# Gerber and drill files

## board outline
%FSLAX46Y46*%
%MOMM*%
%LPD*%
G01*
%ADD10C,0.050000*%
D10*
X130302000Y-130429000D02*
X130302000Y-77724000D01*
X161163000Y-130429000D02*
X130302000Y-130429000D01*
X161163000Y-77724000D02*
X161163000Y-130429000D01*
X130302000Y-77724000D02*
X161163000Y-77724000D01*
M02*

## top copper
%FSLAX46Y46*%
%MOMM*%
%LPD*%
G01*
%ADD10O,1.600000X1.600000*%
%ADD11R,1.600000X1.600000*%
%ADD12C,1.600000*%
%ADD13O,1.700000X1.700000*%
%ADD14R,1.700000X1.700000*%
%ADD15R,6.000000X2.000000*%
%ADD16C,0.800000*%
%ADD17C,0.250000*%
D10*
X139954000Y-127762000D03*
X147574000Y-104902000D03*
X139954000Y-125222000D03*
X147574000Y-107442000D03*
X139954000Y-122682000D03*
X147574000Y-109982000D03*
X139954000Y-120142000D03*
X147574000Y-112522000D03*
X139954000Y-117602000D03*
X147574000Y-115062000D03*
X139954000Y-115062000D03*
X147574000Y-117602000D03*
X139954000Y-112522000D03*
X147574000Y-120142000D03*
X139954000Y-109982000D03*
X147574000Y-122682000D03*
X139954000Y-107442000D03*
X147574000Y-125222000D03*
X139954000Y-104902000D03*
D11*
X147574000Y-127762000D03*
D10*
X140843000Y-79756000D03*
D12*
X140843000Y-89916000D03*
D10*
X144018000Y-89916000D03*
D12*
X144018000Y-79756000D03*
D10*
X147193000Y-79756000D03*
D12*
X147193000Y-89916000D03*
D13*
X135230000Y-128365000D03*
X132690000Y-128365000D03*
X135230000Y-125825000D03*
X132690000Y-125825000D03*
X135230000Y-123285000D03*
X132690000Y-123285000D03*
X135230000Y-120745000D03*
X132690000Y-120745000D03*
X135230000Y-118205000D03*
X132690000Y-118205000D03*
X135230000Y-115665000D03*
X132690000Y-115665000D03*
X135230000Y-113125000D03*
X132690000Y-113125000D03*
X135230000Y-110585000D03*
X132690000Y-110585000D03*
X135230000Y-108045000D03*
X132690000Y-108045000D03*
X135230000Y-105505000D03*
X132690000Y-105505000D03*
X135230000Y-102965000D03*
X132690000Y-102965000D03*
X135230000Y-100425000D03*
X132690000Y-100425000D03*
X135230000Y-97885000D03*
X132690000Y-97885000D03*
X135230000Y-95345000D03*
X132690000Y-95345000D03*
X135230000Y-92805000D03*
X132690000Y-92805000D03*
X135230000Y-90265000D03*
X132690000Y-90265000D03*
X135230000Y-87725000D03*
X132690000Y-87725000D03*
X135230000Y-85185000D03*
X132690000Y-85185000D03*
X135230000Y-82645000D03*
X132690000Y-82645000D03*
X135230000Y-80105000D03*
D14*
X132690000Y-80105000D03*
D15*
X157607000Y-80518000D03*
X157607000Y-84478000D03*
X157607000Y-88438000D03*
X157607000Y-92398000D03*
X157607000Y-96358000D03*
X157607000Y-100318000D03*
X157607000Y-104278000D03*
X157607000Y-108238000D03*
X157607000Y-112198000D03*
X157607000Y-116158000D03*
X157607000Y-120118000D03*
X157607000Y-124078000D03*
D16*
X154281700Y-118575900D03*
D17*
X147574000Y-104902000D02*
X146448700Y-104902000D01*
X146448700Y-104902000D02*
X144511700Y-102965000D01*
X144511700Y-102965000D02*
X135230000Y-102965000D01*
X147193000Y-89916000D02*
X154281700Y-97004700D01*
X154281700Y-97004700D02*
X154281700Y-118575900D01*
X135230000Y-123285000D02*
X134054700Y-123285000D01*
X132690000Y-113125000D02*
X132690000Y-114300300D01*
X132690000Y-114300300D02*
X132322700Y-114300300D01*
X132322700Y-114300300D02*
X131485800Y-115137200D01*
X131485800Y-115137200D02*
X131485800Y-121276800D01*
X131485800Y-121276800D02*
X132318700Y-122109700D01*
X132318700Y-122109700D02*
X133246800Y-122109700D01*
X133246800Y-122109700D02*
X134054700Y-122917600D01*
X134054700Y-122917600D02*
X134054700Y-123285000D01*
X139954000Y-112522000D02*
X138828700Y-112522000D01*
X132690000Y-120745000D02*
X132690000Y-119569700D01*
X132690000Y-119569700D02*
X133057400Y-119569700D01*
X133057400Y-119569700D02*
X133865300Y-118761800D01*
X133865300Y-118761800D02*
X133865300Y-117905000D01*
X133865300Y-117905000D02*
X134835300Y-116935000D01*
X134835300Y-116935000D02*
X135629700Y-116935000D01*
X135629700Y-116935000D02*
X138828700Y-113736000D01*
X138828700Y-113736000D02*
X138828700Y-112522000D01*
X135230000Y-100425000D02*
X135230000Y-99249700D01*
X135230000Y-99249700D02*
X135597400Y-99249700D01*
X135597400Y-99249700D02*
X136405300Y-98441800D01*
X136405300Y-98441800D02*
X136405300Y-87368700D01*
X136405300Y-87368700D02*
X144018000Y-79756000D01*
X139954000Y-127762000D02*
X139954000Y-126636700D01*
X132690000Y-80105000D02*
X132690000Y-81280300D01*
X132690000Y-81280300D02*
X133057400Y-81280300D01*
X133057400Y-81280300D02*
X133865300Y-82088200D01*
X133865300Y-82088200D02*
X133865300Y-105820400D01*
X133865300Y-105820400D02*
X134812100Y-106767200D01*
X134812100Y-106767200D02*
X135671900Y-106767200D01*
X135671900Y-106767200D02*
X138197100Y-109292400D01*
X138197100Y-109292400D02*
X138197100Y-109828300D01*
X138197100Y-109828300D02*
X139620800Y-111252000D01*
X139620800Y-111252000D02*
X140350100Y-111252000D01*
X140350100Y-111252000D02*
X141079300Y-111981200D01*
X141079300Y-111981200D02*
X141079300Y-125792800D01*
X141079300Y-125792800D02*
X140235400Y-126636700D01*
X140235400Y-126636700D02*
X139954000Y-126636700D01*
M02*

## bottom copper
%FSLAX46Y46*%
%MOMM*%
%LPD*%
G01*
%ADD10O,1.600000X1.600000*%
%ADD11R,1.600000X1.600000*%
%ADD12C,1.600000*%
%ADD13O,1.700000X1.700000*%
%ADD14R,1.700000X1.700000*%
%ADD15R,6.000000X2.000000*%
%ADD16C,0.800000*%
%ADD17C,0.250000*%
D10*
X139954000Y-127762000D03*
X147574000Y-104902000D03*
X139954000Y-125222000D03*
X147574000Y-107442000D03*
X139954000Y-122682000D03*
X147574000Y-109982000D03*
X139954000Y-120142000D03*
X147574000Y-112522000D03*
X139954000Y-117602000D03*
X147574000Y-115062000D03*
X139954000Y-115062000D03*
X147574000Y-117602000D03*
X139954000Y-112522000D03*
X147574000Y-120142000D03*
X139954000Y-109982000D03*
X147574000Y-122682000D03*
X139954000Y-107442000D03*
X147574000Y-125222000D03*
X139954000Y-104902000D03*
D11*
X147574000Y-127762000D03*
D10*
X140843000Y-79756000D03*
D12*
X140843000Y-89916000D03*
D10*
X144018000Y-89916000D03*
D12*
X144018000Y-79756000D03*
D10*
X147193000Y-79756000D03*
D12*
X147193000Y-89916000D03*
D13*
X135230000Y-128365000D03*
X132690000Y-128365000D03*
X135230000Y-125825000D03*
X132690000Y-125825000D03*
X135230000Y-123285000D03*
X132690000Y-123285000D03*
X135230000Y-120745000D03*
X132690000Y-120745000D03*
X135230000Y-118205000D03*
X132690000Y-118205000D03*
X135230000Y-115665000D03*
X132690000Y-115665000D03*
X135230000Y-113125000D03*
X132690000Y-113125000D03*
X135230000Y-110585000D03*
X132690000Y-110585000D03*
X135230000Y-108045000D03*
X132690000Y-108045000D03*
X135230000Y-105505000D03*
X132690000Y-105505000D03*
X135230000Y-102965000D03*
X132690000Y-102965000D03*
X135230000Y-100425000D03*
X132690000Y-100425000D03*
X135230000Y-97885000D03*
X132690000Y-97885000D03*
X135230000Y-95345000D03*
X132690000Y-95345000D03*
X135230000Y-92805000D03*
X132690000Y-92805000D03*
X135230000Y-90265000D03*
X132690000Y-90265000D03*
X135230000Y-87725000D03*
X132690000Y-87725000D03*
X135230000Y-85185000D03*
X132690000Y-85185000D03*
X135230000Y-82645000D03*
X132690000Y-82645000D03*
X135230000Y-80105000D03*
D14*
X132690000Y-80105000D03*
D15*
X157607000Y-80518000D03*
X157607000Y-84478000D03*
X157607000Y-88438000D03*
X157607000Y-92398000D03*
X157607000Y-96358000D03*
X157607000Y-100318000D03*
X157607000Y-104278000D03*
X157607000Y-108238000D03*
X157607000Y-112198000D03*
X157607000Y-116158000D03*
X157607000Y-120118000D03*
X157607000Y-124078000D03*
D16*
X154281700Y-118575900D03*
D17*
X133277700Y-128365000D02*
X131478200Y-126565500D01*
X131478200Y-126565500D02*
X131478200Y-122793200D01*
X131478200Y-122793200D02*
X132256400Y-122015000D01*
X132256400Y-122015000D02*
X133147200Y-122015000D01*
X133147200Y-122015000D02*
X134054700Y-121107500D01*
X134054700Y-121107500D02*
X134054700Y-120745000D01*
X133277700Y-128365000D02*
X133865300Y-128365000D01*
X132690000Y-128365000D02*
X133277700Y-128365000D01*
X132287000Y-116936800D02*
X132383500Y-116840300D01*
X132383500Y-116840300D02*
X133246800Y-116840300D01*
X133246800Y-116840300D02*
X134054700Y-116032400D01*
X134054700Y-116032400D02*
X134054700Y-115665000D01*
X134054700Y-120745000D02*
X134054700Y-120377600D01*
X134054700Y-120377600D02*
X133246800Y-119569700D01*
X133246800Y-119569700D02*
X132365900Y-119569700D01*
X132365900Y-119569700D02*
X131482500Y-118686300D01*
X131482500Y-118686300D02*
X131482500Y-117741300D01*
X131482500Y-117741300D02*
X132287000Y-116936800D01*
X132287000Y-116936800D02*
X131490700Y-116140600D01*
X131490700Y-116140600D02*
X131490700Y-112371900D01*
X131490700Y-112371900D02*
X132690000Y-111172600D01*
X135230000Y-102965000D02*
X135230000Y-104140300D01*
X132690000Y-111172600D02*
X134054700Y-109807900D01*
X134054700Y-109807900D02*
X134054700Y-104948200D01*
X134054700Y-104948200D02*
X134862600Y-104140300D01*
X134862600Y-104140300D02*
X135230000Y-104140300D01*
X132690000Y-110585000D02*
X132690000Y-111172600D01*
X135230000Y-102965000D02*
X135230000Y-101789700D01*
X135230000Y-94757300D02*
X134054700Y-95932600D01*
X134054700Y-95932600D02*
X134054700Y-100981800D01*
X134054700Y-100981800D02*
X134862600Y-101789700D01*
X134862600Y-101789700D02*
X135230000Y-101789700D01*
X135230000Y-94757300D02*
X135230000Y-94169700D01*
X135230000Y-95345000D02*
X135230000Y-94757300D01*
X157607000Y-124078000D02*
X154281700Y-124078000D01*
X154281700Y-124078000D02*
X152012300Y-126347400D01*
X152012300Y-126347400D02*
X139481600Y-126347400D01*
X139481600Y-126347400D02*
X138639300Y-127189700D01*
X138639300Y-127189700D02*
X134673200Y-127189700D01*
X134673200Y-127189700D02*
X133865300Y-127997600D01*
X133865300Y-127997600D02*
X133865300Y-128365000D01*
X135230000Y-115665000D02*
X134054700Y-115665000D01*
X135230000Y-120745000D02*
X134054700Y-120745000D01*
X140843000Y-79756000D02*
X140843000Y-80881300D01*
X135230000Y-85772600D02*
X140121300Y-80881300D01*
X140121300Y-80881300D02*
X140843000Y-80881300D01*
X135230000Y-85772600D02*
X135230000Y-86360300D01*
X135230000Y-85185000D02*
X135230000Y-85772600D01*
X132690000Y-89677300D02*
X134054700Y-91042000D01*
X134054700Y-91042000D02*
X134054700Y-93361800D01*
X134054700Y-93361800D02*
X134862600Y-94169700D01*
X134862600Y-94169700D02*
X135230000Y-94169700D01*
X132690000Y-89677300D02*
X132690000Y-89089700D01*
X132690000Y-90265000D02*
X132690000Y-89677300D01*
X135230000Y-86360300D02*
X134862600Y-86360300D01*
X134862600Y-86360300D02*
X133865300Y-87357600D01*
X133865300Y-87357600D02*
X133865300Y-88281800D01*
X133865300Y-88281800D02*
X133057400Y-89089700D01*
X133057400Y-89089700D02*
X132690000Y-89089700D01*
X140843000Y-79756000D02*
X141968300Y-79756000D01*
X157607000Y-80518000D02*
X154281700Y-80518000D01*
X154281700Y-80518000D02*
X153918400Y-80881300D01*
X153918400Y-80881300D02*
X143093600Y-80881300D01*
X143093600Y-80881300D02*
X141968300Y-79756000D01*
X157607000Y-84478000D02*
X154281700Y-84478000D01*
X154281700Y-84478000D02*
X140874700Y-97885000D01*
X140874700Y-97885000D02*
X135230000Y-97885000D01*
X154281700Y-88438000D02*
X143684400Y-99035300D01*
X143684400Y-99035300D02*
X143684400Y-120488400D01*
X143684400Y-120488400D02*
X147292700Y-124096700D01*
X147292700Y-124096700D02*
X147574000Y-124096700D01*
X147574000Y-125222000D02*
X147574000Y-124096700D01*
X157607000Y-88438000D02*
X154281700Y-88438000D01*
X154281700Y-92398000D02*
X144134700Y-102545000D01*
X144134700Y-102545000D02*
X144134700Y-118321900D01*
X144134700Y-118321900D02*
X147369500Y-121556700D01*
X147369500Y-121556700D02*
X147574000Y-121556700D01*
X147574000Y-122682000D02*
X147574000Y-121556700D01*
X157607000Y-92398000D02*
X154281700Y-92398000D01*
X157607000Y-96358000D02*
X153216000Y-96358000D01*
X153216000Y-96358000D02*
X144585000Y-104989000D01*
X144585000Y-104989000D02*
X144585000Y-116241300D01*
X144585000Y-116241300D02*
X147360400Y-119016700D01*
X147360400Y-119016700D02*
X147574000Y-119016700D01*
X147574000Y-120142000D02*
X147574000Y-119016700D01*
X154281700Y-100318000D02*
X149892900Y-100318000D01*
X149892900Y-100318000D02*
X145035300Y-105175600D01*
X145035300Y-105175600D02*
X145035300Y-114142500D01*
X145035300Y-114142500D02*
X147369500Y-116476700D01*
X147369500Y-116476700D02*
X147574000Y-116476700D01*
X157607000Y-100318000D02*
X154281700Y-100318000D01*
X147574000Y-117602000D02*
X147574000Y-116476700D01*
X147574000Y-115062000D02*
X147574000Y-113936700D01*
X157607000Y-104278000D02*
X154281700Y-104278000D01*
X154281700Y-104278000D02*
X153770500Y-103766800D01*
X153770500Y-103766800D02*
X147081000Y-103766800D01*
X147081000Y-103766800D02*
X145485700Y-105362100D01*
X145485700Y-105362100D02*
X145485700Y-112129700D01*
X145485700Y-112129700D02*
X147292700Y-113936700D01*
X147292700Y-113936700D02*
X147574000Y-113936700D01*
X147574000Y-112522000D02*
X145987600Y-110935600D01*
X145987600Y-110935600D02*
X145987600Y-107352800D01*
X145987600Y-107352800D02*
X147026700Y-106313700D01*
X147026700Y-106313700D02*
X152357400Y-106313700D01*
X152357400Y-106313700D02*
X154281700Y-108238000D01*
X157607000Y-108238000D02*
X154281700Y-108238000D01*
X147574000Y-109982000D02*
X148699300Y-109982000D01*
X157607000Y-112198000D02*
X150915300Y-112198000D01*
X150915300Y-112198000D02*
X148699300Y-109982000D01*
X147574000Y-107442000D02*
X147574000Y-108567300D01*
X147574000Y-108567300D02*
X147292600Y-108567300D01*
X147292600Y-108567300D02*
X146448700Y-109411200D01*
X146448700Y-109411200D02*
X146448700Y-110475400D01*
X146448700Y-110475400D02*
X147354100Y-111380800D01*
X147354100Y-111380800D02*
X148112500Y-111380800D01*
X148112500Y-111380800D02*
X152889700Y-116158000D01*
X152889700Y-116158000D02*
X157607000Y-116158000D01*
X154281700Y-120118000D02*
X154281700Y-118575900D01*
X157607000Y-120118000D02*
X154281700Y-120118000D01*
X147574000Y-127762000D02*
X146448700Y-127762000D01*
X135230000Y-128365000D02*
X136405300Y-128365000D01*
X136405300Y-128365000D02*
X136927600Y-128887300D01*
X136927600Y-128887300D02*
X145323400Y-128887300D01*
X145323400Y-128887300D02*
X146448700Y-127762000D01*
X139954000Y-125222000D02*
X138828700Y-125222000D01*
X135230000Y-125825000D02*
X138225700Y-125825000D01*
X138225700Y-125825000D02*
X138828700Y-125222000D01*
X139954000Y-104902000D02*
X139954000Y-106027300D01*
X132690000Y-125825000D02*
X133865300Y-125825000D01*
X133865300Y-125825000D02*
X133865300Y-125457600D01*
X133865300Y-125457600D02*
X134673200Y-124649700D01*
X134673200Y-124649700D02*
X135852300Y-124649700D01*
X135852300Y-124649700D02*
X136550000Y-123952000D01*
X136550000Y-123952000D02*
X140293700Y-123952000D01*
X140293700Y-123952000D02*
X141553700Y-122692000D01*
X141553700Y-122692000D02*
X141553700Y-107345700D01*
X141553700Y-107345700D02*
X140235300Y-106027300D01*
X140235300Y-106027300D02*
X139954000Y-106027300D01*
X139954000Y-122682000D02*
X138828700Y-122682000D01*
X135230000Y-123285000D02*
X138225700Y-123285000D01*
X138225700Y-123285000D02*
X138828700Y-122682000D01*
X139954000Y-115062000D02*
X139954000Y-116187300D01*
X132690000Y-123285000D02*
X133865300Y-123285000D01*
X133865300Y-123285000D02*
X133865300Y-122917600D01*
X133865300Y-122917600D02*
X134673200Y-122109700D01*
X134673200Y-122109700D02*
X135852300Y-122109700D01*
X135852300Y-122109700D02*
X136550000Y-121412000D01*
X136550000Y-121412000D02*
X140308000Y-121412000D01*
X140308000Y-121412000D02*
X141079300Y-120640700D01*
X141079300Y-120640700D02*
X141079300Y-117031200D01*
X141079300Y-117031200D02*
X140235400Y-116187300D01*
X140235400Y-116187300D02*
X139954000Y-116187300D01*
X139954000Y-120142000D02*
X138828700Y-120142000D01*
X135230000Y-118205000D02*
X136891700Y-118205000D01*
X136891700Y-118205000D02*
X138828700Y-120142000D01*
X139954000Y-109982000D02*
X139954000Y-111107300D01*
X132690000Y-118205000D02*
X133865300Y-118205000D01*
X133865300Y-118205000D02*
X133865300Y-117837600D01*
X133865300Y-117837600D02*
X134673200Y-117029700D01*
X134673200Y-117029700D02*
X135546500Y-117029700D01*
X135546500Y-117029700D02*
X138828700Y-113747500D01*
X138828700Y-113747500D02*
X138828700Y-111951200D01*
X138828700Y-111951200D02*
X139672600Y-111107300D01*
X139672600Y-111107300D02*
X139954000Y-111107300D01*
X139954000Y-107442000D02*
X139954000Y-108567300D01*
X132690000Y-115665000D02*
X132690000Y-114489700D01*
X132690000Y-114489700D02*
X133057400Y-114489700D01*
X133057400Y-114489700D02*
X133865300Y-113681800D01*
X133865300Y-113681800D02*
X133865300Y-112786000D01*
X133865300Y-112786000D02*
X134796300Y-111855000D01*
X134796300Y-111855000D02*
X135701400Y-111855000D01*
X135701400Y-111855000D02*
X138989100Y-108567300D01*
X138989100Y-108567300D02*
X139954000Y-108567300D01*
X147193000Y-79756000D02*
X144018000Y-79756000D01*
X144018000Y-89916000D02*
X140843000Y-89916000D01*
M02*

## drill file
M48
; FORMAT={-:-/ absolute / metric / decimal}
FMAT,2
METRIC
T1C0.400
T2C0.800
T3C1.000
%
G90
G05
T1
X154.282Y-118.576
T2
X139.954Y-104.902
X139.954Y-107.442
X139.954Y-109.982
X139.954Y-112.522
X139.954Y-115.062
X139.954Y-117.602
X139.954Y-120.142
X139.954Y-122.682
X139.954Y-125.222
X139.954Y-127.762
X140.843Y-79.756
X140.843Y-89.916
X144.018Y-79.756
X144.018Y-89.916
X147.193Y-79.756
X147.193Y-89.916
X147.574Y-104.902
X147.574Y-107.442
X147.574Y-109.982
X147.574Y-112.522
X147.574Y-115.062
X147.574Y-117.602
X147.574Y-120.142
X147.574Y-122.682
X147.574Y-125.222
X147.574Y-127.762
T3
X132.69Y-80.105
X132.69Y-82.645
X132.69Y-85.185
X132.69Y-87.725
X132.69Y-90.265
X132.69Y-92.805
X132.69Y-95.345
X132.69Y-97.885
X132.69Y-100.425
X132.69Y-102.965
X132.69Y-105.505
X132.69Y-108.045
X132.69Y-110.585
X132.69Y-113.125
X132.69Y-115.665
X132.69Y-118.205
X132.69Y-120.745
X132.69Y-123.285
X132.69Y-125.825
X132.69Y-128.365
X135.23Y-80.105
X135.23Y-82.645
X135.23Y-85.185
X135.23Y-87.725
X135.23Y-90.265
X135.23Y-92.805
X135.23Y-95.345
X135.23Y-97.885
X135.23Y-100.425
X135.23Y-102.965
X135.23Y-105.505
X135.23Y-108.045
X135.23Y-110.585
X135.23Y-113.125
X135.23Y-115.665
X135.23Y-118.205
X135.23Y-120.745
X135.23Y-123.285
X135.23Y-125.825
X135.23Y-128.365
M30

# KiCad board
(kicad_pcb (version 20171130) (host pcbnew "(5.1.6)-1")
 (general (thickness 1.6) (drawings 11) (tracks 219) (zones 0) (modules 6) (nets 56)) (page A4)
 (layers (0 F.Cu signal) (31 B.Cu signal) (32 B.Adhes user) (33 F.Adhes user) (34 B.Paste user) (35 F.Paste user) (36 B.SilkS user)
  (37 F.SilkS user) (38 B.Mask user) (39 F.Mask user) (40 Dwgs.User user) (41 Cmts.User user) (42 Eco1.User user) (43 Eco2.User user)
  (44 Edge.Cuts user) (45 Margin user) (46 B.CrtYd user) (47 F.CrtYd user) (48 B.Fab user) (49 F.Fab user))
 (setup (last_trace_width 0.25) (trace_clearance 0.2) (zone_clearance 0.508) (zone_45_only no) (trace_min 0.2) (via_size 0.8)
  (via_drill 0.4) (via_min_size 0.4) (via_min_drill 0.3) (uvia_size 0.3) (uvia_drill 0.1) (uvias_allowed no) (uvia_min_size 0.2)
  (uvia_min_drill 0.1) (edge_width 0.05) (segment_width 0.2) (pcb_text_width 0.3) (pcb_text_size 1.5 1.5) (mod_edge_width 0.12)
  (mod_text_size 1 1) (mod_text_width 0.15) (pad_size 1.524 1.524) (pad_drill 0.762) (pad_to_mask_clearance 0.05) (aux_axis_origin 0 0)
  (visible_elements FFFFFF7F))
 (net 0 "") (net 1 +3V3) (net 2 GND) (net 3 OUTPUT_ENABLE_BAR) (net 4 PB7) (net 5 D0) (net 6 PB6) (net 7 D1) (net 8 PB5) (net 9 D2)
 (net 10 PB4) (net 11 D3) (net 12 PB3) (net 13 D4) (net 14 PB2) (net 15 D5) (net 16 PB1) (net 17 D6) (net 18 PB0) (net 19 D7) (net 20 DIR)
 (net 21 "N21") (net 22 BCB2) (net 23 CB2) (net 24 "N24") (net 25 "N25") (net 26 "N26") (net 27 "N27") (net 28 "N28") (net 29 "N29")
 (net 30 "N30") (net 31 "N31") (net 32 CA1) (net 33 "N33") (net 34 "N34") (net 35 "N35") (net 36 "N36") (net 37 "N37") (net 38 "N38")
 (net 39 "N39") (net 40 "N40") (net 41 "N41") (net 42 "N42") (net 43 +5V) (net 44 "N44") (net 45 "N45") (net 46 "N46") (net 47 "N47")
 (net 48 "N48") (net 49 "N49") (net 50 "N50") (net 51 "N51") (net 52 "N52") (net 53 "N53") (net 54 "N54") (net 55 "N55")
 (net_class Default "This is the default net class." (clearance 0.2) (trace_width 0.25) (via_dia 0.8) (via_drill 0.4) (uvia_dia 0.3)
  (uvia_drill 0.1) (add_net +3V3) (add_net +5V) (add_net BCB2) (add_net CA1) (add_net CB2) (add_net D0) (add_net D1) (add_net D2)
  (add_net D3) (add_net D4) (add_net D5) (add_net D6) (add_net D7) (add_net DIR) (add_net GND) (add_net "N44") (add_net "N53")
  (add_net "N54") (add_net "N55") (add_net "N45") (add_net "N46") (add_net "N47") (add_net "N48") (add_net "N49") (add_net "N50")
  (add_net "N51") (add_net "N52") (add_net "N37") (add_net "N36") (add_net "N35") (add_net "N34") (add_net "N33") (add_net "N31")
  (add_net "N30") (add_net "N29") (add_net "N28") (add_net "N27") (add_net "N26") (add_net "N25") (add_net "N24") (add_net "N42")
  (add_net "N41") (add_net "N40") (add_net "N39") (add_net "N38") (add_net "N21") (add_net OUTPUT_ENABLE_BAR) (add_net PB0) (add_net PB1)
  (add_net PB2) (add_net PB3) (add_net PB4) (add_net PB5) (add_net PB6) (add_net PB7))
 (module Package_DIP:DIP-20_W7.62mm (layer F.Cu) (at 147.574 127.762 180)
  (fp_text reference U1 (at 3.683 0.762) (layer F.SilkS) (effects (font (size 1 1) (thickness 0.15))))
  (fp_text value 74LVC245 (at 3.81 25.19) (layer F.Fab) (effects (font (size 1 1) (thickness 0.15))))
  (pad 20 thru_hole oval (at 7.62 0 180) (size 1.6 1.6) (drill 0.8) (layers *.Cu *.Mask) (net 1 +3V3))
  (pad 10 thru_hole oval (at 0 22.86 180) (size 1.6 1.6) (drill 0.8) (layers *.Cu *.Mask) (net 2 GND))
  (pad 19 thru_hole oval (at 7.62 2.54 180) (size 1.6 1.6) (drill 0.8) (layers *.Cu *.Mask) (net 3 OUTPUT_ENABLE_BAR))
  (pad 9 thru_hole oval (at 0 20.32 180) (size 1.6 1.6) (drill 0.8) (layers *.Cu *.Mask) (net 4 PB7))
  (pad 18 thru_hole oval (at 7.62 5.08 180) (size 1.6 1.6) (drill 0.8) (layers *.Cu *.Mask) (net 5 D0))
  (pad 8 thru_hole oval (at 0 17.78 180) (size 1.6 1.6) (drill 0.8) (layers *.Cu *.Mask) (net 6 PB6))
  (pad 17 thru_hole oval (at 7.62 7.62 180) (size 1.6 1.6) (drill 0.8) (layers *.Cu *.Mask) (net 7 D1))
  (pad 7 thru_hole oval (at 0 15.24 180) (size 1.6 1.6) (drill 0.8) (layers *.Cu *.Mask) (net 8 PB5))
  (pad 16 thru_hole oval (at 7.62 10.16 180) (size 1.6 1.6) (drill 0.8) (layers *.Cu *.Mask) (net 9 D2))
  (pad 6 thru_hole oval (at 0 12.7 180) (size 1.6 1.6) (drill 0.8) (layers *.Cu *.Mask) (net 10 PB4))
  (pad 15 thru_hole oval (at 7.62 12.7 180) (size 1.6 1.6) (drill 0.8) (layers *.Cu *.Mask) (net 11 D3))
  (pad 5 thru_hole oval (at 0 10.16 180) (size 1.6 1.6) (drill 0.8) (layers *.Cu *.Mask) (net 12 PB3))
  (pad 14 thru_hole oval (at 7.62 15.24 180) (size 1.6 1.6) (drill 0.8) (layers *.Cu *.Mask) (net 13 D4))
  (pad 4 thru_hole oval (at 0 7.62 180) (size 1.6 1.6) (drill 0.8) (layers *.Cu *.Mask) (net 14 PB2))
  (pad 13 thru_hole oval (at 7.62 17.78 180) (size 1.6 1.6) (drill 0.8) (layers *.Cu *.Mask) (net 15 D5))
  (pad 3 thru_hole oval (at 0 5.08 180) (size 1.6 1.6) (drill 0.8) (layers *.Cu *.Mask) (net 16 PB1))
  (pad 12 thru_hole oval (at 7.62 20.32 180) (size 1.6 1.6) (drill 0.8) (layers *.Cu *.Mask) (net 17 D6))
  (pad 2 thru_hole oval (at 0 2.54 180) (size 1.6 1.6) (drill 0.8) (layers *.Cu *.Mask) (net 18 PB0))
  (pad 11 thru_hole oval (at 7.62 22.86 180) (size 1.6 1.6) (drill 0.8) (layers *.Cu *.Mask) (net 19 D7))
  (pad 1 thru_hole rect (at 0 0 180) (size 1.6 1.6) (drill 0.8) (layers *.Cu *.Mask) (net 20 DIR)))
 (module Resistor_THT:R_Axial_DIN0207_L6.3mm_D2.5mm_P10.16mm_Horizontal (layer F.Cu) (at 140.843 89.916 90)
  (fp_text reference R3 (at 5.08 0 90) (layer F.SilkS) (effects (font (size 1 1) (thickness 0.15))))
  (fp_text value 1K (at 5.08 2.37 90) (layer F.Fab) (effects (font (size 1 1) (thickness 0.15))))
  (pad 2 thru_hole oval (at 10.16 0 90) (size 1.6 1.6) (drill 0.8) (layers *.Cu *.Mask) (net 2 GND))
  (pad 1 thru_hole circle (at 0 0 90) (size 1.6 1.6) (drill 0.8) (layers *.Cu *.Mask) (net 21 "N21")))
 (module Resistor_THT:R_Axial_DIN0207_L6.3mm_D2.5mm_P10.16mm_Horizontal (layer F.Cu) (at 144.018 79.756 270)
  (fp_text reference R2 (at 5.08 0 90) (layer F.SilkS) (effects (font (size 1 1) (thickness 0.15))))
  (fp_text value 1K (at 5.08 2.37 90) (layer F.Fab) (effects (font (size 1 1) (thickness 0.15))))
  (pad 2 thru_hole oval (at 10.16 0 270) (size 1.6 1.6) (drill 0.8) (layers *.Cu *.Mask) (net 21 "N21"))
  (pad 1 thru_hole circle (at 0 0 270) (size 1.6 1.6) (drill 0.8) (layers *.Cu *.Mask) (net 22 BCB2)))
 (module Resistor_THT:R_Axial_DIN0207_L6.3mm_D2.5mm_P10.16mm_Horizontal (layer F.Cu) (at 147.193 89.916 90)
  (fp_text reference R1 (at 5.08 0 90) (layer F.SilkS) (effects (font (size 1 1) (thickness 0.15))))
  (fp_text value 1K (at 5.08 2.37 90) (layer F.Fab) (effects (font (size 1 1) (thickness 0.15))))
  (pad 2 thru_hole oval (at 10.16 0 90) (size 1.6 1.6) (drill 0.8) (layers *.Cu *.Mask) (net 22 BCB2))
  (pad 1 thru_hole circle (at 0 0 90) (size 1.6 1.6) (drill 0.8) (layers *.Cu *.Mask) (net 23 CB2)))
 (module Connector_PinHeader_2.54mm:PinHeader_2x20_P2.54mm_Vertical (layer F.Cu) (at 132.69 80.105)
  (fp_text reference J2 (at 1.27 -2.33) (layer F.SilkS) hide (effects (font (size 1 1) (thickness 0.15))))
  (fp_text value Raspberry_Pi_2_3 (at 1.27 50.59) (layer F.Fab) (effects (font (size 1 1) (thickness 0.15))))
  (pad 40 thru_hole oval (at 2.54 48.26) (size 1.7 1.7) (drill 1) (layers *.Cu *.Mask) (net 20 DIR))
  (pad 39 thru_hole oval (at 0 48.26) (size 1.7 1.7) (drill 1) (layers *.Cu *.Mask) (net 2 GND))
  (pad 38 thru_hole oval (at 2.54 45.72) (size 1.7 1.7) (drill 1) (layers *.Cu *.Mask) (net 3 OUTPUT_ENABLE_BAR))
  (pad 37 thru_hole oval (at 0 45.72) (size 1.7 1.7) (drill 1) (layers *.Cu *.Mask) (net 19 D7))
  (pad 36 thru_hole oval (at 2.54 43.18) (size 1.7 1.7) (drill 1) (layers *.Cu *.Mask) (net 5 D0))
  (pad 35 thru_hole oval (at 0 43.18) (size 1.7 1.7) (drill 1) (layers *.Cu *.Mask) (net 11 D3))
  (pad 34 thru_hole oval (at 2.54 40.64) (size 1.7 1.7) (drill 1) (layers *.Cu *.Mask) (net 2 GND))
  (pad 33 thru_hole oval (at 0 40.64) (size 1.7 1.7) (drill 1) (layers *.Cu *.Mask) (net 13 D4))
  (pad 32 thru_hole oval (at 2.54 38.1) (size 1.7 1.7) (drill 1) (layers *.Cu *.Mask) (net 7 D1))
  (pad 31 thru_hole oval (at 0 38.1) (size 1.7 1.7) (drill 1) (layers *.Cu *.Mask) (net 15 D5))
  (pad 30 thru_hole oval (at 2.54 35.56) (size 1.7 1.7) (drill 1) (layers *.Cu *.Mask) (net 2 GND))
  (pad 29 thru_hole oval (at 0 35.56) (size 1.7 1.7) (drill 1) (layers *.Cu *.Mask) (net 17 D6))
  (pad 28 thru_hole oval (at 2.54 33.02) (size 1.7 1.7) (drill 1) (layers *.Cu *.Mask) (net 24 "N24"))
  (pad 27 thru_hole oval (at 0 33.02) (size 1.7 1.7) (drill 1) (layers *.Cu *.Mask) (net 5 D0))
  (pad 26 thru_hole oval (at 2.54 30.48) (size 1.7 1.7) (drill 1) (layers *.Cu *.Mask) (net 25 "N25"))
  (pad 25 thru_hole oval (at 0 30.48) (size 1.7 1.7) (drill 1) (layers *.Cu *.Mask) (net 2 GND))
  (pad 24 thru_hole oval (at 2.54 27.94) (size 1.7 1.7) (drill 1) (layers *.Cu *.Mask) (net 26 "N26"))
  (pad 23 thru_hole oval (at 0 27.94) (size 1.7 1.7) (drill 1) (layers *.Cu *.Mask) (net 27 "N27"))
  (pad 22 thru_hole oval (at 2.54 25.4) (size 1.7 1.7) (drill 1) (layers *.Cu *.Mask) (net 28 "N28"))
  (pad 21 thru_hole oval (at 0 25.4) (size 1.7 1.7) (drill 1) (layers *.Cu *.Mask) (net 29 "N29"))
  (pad 20 thru_hole oval (at 2.54 22.86) (size 1.7 1.7) (drill 1) (layers *.Cu *.Mask) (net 2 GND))
  (pad 19 thru_hole oval (at 0 22.86) (size 1.7 1.7) (drill 1) (layers *.Cu *.Mask) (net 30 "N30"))
  (pad 18 thru_hole oval (at 2.54 20.32) (size 1.7 1.7) (drill 1) (layers *.Cu *.Mask) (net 22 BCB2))
  (pad 17 thru_hole oval (at 0 20.32) (size 1.7 1.7) (drill 1) (layers *.Cu *.Mask) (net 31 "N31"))
  (pad 16 thru_hole oval (at 2.54 17.78) (size 1.7 1.7) (drill 1) (layers *.Cu *.Mask) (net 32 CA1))
  (pad 15 thru_hole oval (at 0 17.78) (size 1.7 1.7) (drill 1) (layers *.Cu *.Mask) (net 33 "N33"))
  (pad 14 thru_hole oval (at 2.54 15.24) (size 1.7 1.7) (drill 1) (layers *.Cu *.Mask) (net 2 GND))
  (pad 13 thru_hole oval (at 0 15.24) (size 1.7 1.7) (drill 1) (layers *.Cu *.Mask) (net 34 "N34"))
  (pad 12 thru_hole oval (at 2.54 12.7) (size 1.7 1.7) (drill 1) (layers *.Cu *.Mask) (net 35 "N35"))
  (pad 11 thru_hole oval (at 0 12.7) (size 1.7 1.7) (drill 1) (layers *.Cu *.Mask) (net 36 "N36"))
  (pad 10 thru_hole oval (at 2.54 10.16) (size 1.7 1.7) (drill 1) (layers *.Cu *.Mask) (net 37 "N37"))
  (pad 9 thru_hole oval (at 0 10.16) (size 1.7 1.7) (drill 1) (layers *.Cu *.Mask) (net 2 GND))
  (pad 8 thru_hole oval (at 2.54 7.62) (size 1.7 1.7) (drill 1) (layers *.Cu *.Mask) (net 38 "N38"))
  (pad 7 thru_hole oval (at 0 7.62) (size 1.7 1.7) (drill 1) (layers *.Cu *.Mask) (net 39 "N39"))
  (pad 6 thru_hole oval (at 2.54 5.08) (size 1.7 1.7) (drill 1) (layers *.Cu *.Mask) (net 2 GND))
  (pad 5 thru_hole oval (at 0 5.08) (size 1.7 1.7) (drill 1) (layers *.Cu *.Mask) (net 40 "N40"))
  (pad 4 thru_hole oval (at 2.54 2.54) (size 1.7 1.7) (drill 1) (layers *.Cu *.Mask) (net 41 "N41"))
  (pad 3 thru_hole oval (at 0 2.54) (size 1.7 1.7) (drill 1) (layers *.Cu *.Mask) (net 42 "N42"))
  (pad 2 thru_hole oval (at 2.54 0) (size 1.7 1.7) (drill 1) (layers *.Cu *.Mask) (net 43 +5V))
  (pad 1 thru_hole rect (at 0 0) (size 1.7 1.7) (drill 1) (layers *.Cu *.Mask) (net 1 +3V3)))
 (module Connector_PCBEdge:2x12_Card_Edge (layer F.Cu) (at 157.607 80.518 270)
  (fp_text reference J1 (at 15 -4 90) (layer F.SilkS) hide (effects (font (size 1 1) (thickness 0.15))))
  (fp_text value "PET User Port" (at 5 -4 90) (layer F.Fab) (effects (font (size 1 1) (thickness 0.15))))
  (pad 1 smd rect (at 0 0 270) (size 2 6) (layers F.Cu F.Paste F.Mask) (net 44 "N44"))
  (pad 2 smd rect (at 3.96 0 270) (size 2 6) (layers F.Cu F.Paste F.Mask) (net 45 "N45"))
  (pad 3 smd rect (at 7.92 0 270) (size 2 6) (layers F.Cu F.Paste F.Mask) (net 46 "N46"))
  (pad 4 smd rect (at 11.88 0 270) (size 2 6) (layers F.Cu F.Paste F.Mask) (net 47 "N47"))
  (pad 5 smd rect (at 15.84 0 270) (size 2 6) (layers F.Cu F.Paste F.Mask) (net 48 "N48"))
  (pad 6 smd rect (at 19.8 0 270) (size 2 6) (layers F.Cu F.Paste F.Mask) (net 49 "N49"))
  (pad 7 smd rect (at 23.76 0 270) (size 2 6) (layers F.Cu F.Paste F.Mask) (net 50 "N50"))
  (pad 8 smd rect (at 27.72 0 270) (size 2 6) (layers F.Cu F.Paste F.Mask) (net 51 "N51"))
  (pad 9 smd rect (at 31.68 0 270) (size 2 6) (layers F.Cu F.Paste F.Mask) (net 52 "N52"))
  (pad 10 smd rect (at 35.64 0 270) (size 2 6) (layers F.Cu F.Paste F.Mask) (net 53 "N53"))
  (pad 11 smd rect (at 39.6 0 270) (size 2 6) (layers F.Cu F.Paste F.Mask) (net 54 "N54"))
  (pad 12 smd rect (at 43.56 0 270) (size 2 6) (layers F.Cu F.Paste F.Mask) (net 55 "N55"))
  (pad 13 smd rect (at 0 0 270) (size 2 6) (layers B.Cu B.Paste B.Mask) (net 2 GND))
  (pad 14 smd rect (at 3.96 0 270) (size 2 6) (layers B.Cu B.Paste B.Mask) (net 32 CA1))
  (pad 15 smd rect (at 7.92 0 270) (size 2 6) (layers B.Cu B.Paste B.Mask) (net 18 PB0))
  (pad 16 smd rect (at 11.88 0 270) (size 2 6) (layers B.Cu B.Paste B.Mask) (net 16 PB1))
  (pad 17 smd rect (at 15.84 0 270) (size 2 6) (layers B.Cu B.Paste B.Mask) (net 14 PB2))
  (pad 18 smd rect (at 19.8 0 270) (size 2 6) (layers B.Cu B.Paste B.Mask) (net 12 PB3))
  (pad 19 smd rect (at 23.76 0 270) (size 2 6) (layers B.Cu B.Paste B.Mask) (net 10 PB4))
  (pad 20 smd rect (at 27.72 0 270) (size 2 6) (layers B.Cu B.Paste B.Mask) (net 8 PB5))
  (pad 21 smd rect (at 31.68 0 270) (size 2 6) (layers B.Cu B.Paste B.Mask) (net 6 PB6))
  (pad 22 smd rect (at 35.64 0 270) (size 2 6) (layers B.Cu B.Paste B.Mask) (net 4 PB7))
  (pad 23 smd rect (at 39.6 0 270) (size 2 6) (layers B.Cu B.Paste B.Mask) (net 23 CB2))
  (pad 24 smd rect (at 43.56 0 270) (size 2 6) (layers B.Cu B.Paste B.Mask) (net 2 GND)))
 (gr_line (start 130.302 130.429) (end 130.302 77.724) (layer Edge.Cuts) (width 0.05))
 (gr_line (start 161.163 130.429) (end 130.302 130.429) (layer Edge.Cuts) (width 0.05))
 (gr_line (start 161.163 77.724) (end 161.163 130.429) (layer Edge.Cuts) (width 0.05))
 (gr_line (start 130.302 77.724) (end 161.163 77.724) (layer Edge.Cuts) (width 0.05))
 (segment (start 133.2777 128.365) (end 131.4782 126.5655) (width 0.25) (layer B.Cu) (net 2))
 (segment (start 131.4782 126.5655) (end 131.4782 122.7932) (width 0.25) (layer B.Cu) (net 2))
 (segment (start 131.4782 122.7932) (end 132.2564 122.015) (width 0.25) (layer B.Cu) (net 2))
 (segment (start 132.2564 122.015) (end 133.1472 122.015) (width 0.25) (layer B.Cu) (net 2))
 (segment (start 133.1472 122.015) (end 134.0547 121.1075) (width 0.25) (layer B.Cu) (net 2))
 (segment (start 134.0547 121.1075) (end 134.0547 120.745) (width 0.25) (layer B.Cu) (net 2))
 (segment (start 133.2777 128.365) (end 133.8653 128.365) (width 0.25) (layer B.Cu) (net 2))
 (segment (start 132.69 128.365) (end 133.2777 128.365) (width 0.25) (layer B.Cu) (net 2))
 (segment (start 132.287 116.9368) (end 132.3835 116.8403) (width 0.25) (layer B.Cu) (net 2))
 (segment (start 132.3835 116.8403) (end 133.2468 116.8403) (width 0.25) (layer B.Cu) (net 2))
 (segment (start 133.2468 116.8403) (end 134.0547 116.0324) (width 0.25) (layer B.Cu) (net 2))
 (segment (start 134.0547 116.0324) (end 134.0547 115.665) (width 0.25) (layer B.Cu) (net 2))
 (segment (start 134.0547 120.745) (end 134.0547 120.3776) (width 0.25) (layer B.Cu) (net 2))
 (segment (start 134.0547 120.3776) (end 133.2468 119.5697) (width 0.25) (layer B.Cu) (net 2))
 (segment (start 133.2468 119.5697) (end 132.3659 119.5697) (width 0.25) (layer B.Cu) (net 2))
 (segment (start 132.3659 119.5697) (end 131.4825 118.6863) (width 0.25) (layer B.Cu) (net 2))
 (segment (start 131.4825 118.6863) (end 131.4825 117.7413) (width 0.25) (layer B.Cu) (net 2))
 (segment (start 131.4825 117.7413) (end 132.287 116.9368) (width 0.25) (layer B.Cu) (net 2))
 (segment (start 132.287 116.9368) (end 131.4907 116.1406) (width 0.25) (layer B.Cu) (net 2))
 (segment (start 131.4907 116.1406) (end 131.4907 112.3719) (width 0.25) (layer B.Cu) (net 2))
 (segment (start 131.4907 112.3719) (end 132.69 111.1726) (width 0.25) (layer B.Cu) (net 2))
 (segment (start 135.23 102.965) (end 135.23 104.1403) (width 0.25) (layer B.Cu) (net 2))
 (segment (start 132.69 111.1726) (end 134.0547 109.8079) (width 0.25) (layer B.Cu) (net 2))
 (segment (start 134.0547 109.8079) (end 134.0547 104.9482) (width 0.25) (layer B.Cu) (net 2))
 (segment (start 134.0547 104.9482) (end 134.8626 104.1403) (width 0.25) (layer B.Cu) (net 2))
 (segment (start 134.8626 104.1403) (end 135.23 104.1403) (width 0.25) (layer B.Cu) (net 2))
 (segment (start 132.69 110.585) (end 132.69 111.1726) (width 0.25) (layer B.Cu) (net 2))
 (segment (start 135.23 102.965) (end 135.23 101.7897) (width 0.25) (layer B.Cu) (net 2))
 (segment (start 135.23 94.7573) (end 134.0547 95.9326) (width 0.25) (layer B.Cu) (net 2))
 (segment (start 134.0547 95.9326) (end 134.0547 100.9818) (width 0.25) (layer B.Cu) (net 2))
 (segment (start 134.0547 100.9818) (end 134.8626 101.7897) (width 0.25) (layer B.Cu) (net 2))
 (segment (start 134.8626 101.7897) (end 135.23 101.7897) (width 0.25) (layer B.Cu) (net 2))
 (segment (start 135.23 94.7573) (end 135.23 94.1697) (width 0.25) (layer B.Cu) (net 2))
 (segment (start 135.23 95.345) (end 135.23 94.7573) (width 0.25) (layer B.Cu) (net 2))
 (segment (start 157.607 124.078) (end 154.2817 124.078) (width 0.25) (layer B.Cu) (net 2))
 (segment (start 154.2817 124.078) (end 152.0123 126.3474) (width 0.25) (layer B.Cu) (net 2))
 (segment (start 152.0123 126.3474) (end 139.4816 126.3474) (width 0.25) (layer B.Cu) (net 2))
 (segment (start 139.4816 126.3474) (end 138.6393 127.1897) (width 0.25) (layer B.Cu) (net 2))
 (segment (start 138.6393 127.1897) (end 134.6732 127.1897) (width 0.25) (layer B.Cu) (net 2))
 (segment (start 134.6732 127.1897) (end 133.8653 127.9976) (width 0.25) (layer B.Cu) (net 2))
 (segment (start 133.8653 127.9976) (end 133.8653 128.365) (width 0.25) (layer B.Cu) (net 2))
 (segment (start 147.574 104.902) (end 146.4487 104.902) (width 0.25) (layer F.Cu) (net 2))
 (segment (start 146.4487 104.902) (end 144.5117 102.965) (width 0.25) (layer F.Cu) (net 2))
 (segment (start 144.5117 102.965) (end 135.23 102.965) (width 0.25) (layer F.Cu) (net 2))
 (segment (start 135.23 115.665) (end 134.0547 115.665) (width 0.25) (layer B.Cu) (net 2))
 (segment (start 135.23 120.745) (end 134.0547 120.745) (width 0.25) (layer B.Cu) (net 2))
 (segment (start 140.843 79.756) (end 140.843 80.8813) (width 0.25) (layer B.Cu) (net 2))
 (segment (start 135.23 85.7726) (end 140.1213 80.8813) (width 0.25) (layer B.Cu) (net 2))
 (segment (start 140.1213 80.8813) (end 140.843 80.8813) (width 0.25) (layer B.Cu) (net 2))
 (segment (start 135.23 85.7726) (end 135.23 86.3603) (width 0.25) (layer B.Cu) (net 2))
 (segment (start 135.23 85.185) (end 135.23 85.7726) (width 0.25) (layer B.Cu) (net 2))
 (segment (start 132.69 89.6773) (end 134.0547 91.042) (width 0.25) (layer B.Cu) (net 2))
 (segment (start 134.0547 91.042) (end 134.0547 93.3618) (width 0.25) (layer B.Cu) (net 2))
 (segment (start 134.0547 93.3618) (end 134.8626 94.1697) (width 0.25) (layer B.Cu) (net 2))
 (segment (start 134.8626 94.1697) (end 135.23 94.1697) (width 0.25) (layer B.Cu) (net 2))
 (segment (start 132.69 89.6773) (end 132.69 89.0897) (width 0.25) (layer B.Cu) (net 2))
 (segment (start 132.69 90.265) (end 132.69 89.6773) (width 0.25) (layer B.Cu) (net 2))
 (segment (start 135.23 86.3603) (end 134.8626 86.3603) (width 0.25) (layer B.Cu) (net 2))
 (segment (start 134.8626 86.3603) (end 133.8653 87.3576) (width 0.25) (layer B.Cu) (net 2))
 (segment (start 133.8653 87.3576) (end 133.8653 88.2818) (width 0.25) (layer B.Cu) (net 2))
 (segment (start 133.8653 88.2818) (end 133.0574 89.0897) (width 0.25) (layer B.Cu) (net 2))
 (segment (start 133.0574 89.0897) (end 132.69 89.0897) (width 0.25) (layer B.Cu) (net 2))
 (segment (start 140.843 79.756) (end 141.9683 79.756) (width 0.25) (layer B.Cu) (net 2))
 (segment (start 157.607 80.518) (end 154.2817 80.518) (width 0.25) (layer B.Cu) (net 2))
 (segment (start 154.2817 80.518) (end 153.9184 80.8813) (width 0.25) (layer B.Cu) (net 2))
 (segment (start 153.9184 80.8813) (end 143.0936 80.8813) (width 0.25) (layer B.Cu) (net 2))
 (segment (start 143.0936 80.8813) (end 141.9683 79.756) (width 0.25) (layer B.Cu) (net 2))
 (segment (start 157.607 84.478) (end 154.2817 84.478) (width 0.25) (layer B.Cu) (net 32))
 (segment (start 154.2817 84.478) (end 140.8747 97.885) (width 0.25) (layer B.Cu) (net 32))
 (segment (start 140.8747 97.885) (end 135.23 97.885) (width 0.25) (layer B.Cu) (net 32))
 (segment (start 154.2817 88.438) (end 143.6844 99.0353) (width 0.25) (layer B.Cu) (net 18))
 (segment (start 143.6844 99.0353) (end 143.6844 120.4884) (width 0.25) (layer B.Cu) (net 18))
 (segment (start 143.6844 120.4884) (end 147.2927 124.0967) (width 0.25) (layer B.Cu) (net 18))
 (segment (start 147.2927 124.0967) (end 147.574 124.0967) (width 0.25) (layer B.Cu) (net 18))
 (segment (start 147.574 125.222) (end 147.574 124.0967) (width 0.25) (layer B.Cu) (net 18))
 (segment (start 157.607 88.438) (end 154.2817 88.438) (width 0.25) (layer B.Cu) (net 18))
 (segment (start 154.2817 92.398) (end 144.1347 102.545) (width 0.25) (layer B.Cu) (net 16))
 (segment (start 144.1347 102.545) (end 144.1347 118.3219) (width 0.25) (layer B.Cu) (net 16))
 (segment (start 144.1347 118.3219) (end 147.3695 121.5567) (width 0.25) (layer B.Cu) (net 16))
 (segment (start 147.3695 121.5567) (end 147.574 121.5567) (width 0.25) (layer B.Cu) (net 16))
 (segment (start 147.574 122.682) (end 147.574 121.5567) (width 0.25) (layer B.Cu) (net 16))
 (segment (start 157.607 92.398) (end 154.2817 92.398) (width 0.25) (layer B.Cu) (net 16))
 (segment (start 157.607 96.358) (end 153.216 96.358) (width 0.25) (layer B.Cu) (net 14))
 (segment (start 153.216 96.358) (end 144.585 104.989) (width 0.25) (layer B.Cu) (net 14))
 (segment (start 144.585 104.989) (end 144.585 116.2413) (width 0.25) (layer B.Cu) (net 14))
 (segment (start 144.585 116.2413) (end 147.3604 119.0167) (width 0.25) (layer B.Cu) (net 14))
 (segment (start 147.3604 119.0167) (end 147.574 119.0167) (width 0.25) (layer B.Cu) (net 14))
 (segment (start 147.574 120.142) (end 147.574 119.0167) (width 0.25) (layer B.Cu) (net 14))
 (segment (start 154.2817 100.318) (end 149.8929 100.318) (width 0.25) (layer B.Cu) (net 12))
 (segment (start 149.8929 100.318) (end 145.0353 105.1756) (width 0.25) (layer B.Cu) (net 12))
 (segment (start 145.0353 105.1756) (end 145.0353 114.1425) (width 0.25) (layer B.Cu) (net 12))
 (segment (start 145.0353 114.1425) (end 147.3695 116.4767) (width 0.25) (layer B.Cu) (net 12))
 (segment (start 147.3695 116.4767) (end 147.574 116.4767) (width 0.25) (layer B.Cu) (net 12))
 (segment (start 157.607 100.318) (end 154.2817 100.318) (width 0.25) (layer B.Cu) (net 12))
 (segment (start 147.574 117.602) (end 147.574 116.4767) (width 0.25) (layer B.Cu) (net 12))
 (segment (start 147.574 115.062) (end 147.574 113.9367) (width 0.25) (layer B.Cu) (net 10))
 (segment (start 157.607 104.278) (end 154.2817 104.278) (width 0.25) (layer B.Cu) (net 10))
 (segment (start 154.2817 104.278) (end 153.7705 103.7668) (width 0.25) (layer B.Cu) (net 10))
 (segment (start 153.7705 103.7668) (end 147.081 103.7668) (width 0.25) (layer B.Cu) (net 10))
 (segment (start 147.081 103.7668) (end 145.4857 105.3621) (width 0.25) (layer B.Cu) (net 10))
 (segment (start 145.4857 105.3621) (end 145.4857 112.1297) (width 0.25) (layer B.Cu) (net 10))
 (segment (start 145.4857 112.1297) (end 147.2927 113.9367) (width 0.25) (layer B.Cu) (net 10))
 (segment (start 147.2927 113.9367) (end 147.574 113.9367) (width 0.25) (layer B.Cu) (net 10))
 (segment (start 147.574 112.522) (end 145.9876 110.9356) (width 0.25) (layer B.Cu) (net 8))
 (segment (start 145.9876 110.9356) (end 145.9876 107.3528) (width 0.25) (layer B.Cu) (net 8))
 (segment (start 145.9876 107.3528) (end 147.0267 106.3137) (width 0.25) (layer B.Cu) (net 8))
 (segment (start 147.0267 106.3137) (end 152.3574 106.3137) (width 0.25) (layer B.Cu) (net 8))
 (segment (start 152.3574 106.3137) (end 154.2817 108.238) (width 0.25) (layer B.Cu) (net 8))
 (segment (start 157.607 108.238) (end 154.2817 108.238) (width 0.25) (layer B.Cu) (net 8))
 (segment (start 147.574 109.982) (end 148.6993 109.982) (width 0.25) (layer B.Cu) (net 6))
 (segment (start 157.607 112.198) (end 150.9153 112.198) (width 0.25) (layer B.Cu) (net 6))
 (segment (start 150.9153 112.198) (end 148.6993 109.982) (width 0.25) (layer B.Cu) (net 6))
 (segment (start 147.574 107.442) (end 147.574 108.5673) (width 0.25) (layer B.Cu) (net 4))
 (segment (start 147.574 108.5673) (end 147.2926 108.5673) (width 0.25) (layer B.Cu) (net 4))
 (segment (start 147.2926 108.5673) (end 146.4487 109.4112) (width 0.25) (layer B.Cu) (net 4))
 (segment (start 146.4487 109.4112) (end 146.4487 110.4754) (width 0.25) (layer B.Cu) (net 4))
 (segment (start 146.4487 110.4754) (end 147.3541 111.3808) (width 0.25) (layer B.Cu) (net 4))
 (segment (start 147.3541 111.3808) (end 148.1125 111.3808) (width 0.25) (layer B.Cu) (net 4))
 (segment (start 148.1125 111.3808) (end 152.8897 116.158) (width 0.25) (layer B.Cu) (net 4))
 (segment (start 152.8897 116.158) (end 157.607 116.158) (width 0.25) (layer B.Cu) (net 4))
 (segment (start 147.193 89.916) (end 154.2817 97.0047) (width 0.25) (layer F.Cu) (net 23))
 (segment (start 154.2817 97.0047) (end 154.2817 118.5759) (width 0.25) (layer F.Cu) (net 23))
 (segment (start 154.2817 120.118) (end 154.2817 118.5759) (width 0.25) (layer B.Cu) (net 23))
 (segment (start 157.607 120.118) (end 154.2817 120.118) (width 0.25) (layer B.Cu) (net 23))
 (via (at 154.2817 118.5759) (size 0.8) (layers F.Cu B.Cu) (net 23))
 (segment (start 147.574 127.762) (end 146.4487 127.762) (width 0.25) (layer B.Cu) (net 20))
 (segment (start 135.23 128.365) (end 136.4053 128.365) (width 0.25) (layer B.Cu) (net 20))
 (segment (start 136.4053 128.365) (end 136.9276 128.8873) (width 0.25) (layer B.Cu) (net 20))
 (segment (start 136.9276 128.8873) (end 145.3234 128.8873) (width 0.25) (layer B.Cu) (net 20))
 (segment (start 145.3234 128.8873) (end 146.4487 127.762) (width 0.25) (layer B.Cu) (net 20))
 (segment (start 139.954 125.222) (end 138.8287 125.222) (width 0.25) (layer B.Cu) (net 3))
 (segment (start 135.23 125.825) (end 138.2257 125.825) (width 0.25) (layer B.Cu) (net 3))
 (segment (start 138.2257 125.825) (end 138.8287 125.222) (width 0.25) (layer B.Cu) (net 3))
 (segment (start 139.954 104.902) (end 139.954 106.0273) (width 0.25) (layer B.Cu) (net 19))
 (segment (start 132.69 125.825) (end 133.8653 125.825) (width 0.25) (layer B.Cu) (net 19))
 (segment (start 133.8653 125.825) (end 133.8653 125.4576) (width 0.25) (layer B.Cu) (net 19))
 (segment (start 133.8653 125.4576) (end 134.6732 124.6497) (width 0.25) (layer B.Cu) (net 19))
 (segment (start 134.6732 124.6497) (end 135.8523 124.6497) (width 0.25) (layer B.Cu) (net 19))
 (segment (start 135.8523 124.6497) (end 136.55 123.952) (width 0.25) (layer B.Cu) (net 19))
 (segment (start 136.55 123.952) (end 140.2937 123.952) (width 0.25) (layer B.Cu) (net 19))
 (segment (start 140.2937 123.952) (end 141.5537 122.692) (width 0.25) (layer B.Cu) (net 19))
 (segment (start 141.5537 122.692) (end 141.5537 107.3457) (width 0.25) (layer B.Cu) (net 19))
 (segment (start 141.5537 107.3457) (end 140.2353 106.0273) (width 0.25) (layer B.Cu) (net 19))
 (segment (start 140.2353 106.0273) (end 139.954 106.0273) (width 0.25) (layer B.Cu) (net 19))
 (segment (start 135.23 123.285) (end 134.0547 123.285) (width 0.25) (layer F.Cu) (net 5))
 (segment (start 132.69 113.125) (end 132.69 114.3003) (width 0.25) (layer F.Cu) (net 5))
 (segment (start 132.69 114.3003) (end 132.3227 114.3003) (width 0.25) (layer F.Cu) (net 5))
 (segment (start 132.3227 114.3003) (end 131.4858 115.1372) (width 0.25) (layer F.Cu) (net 5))
 (segment (start 131.4858 115.1372) (end 131.4858 121.2768) (width 0.25) (layer F.Cu) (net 5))
 (segment (start 131.4858 121.2768) (end 132.3187 122.1097) (width 0.25) (layer F.Cu) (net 5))
 (segment (start 132.3187 122.1097) (end 133.2468 122.1097) (width 0.25) (layer F.Cu) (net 5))
 (segment (start 133.2468 122.1097) (end 134.0547 122.9176) (width 0.25) (layer F.Cu) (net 5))
 (segment (start 134.0547 122.9176) (end 134.0547 123.285) (width 0.25) (layer F.Cu) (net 5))
 (segment (start 139.954 122.682) (end 138.8287 122.682) (width 0.25) (layer B.Cu) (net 5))
 (segment (start 135.23 123.285) (end 138.2257 123.285) (width 0.25) (layer B.Cu) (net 5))
 (segment (start 138.2257 123.285) (end 138.8287 122.682) (width 0.25) (layer B.Cu) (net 5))
 (segment (start 139.954 115.062) (end 139.954 116.1873) (width 0.25) (layer B.Cu) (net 11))
 (segment (start 132.69 123.285) (end 133.8653 123.285) (width 0.25) (layer B.Cu) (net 11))
 (segment (start 133.8653 123.285) (end 133.8653 122.9176) (width 0.25) (layer B.Cu) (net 11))
 (segment (start 133.8653 122.9176) (end 134.6732 122.1097) (width 0.25) (layer B.Cu) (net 11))
 (segment (start 134.6732 122.1097) (end 135.8523 122.1097) (width 0.25) (layer B.Cu) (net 11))
 (segment (start 135.8523 122.1097) (end 136.55 121.412) (width 0.25) (layer B.Cu) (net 11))
 (segment (start 136.55 121.412) (end 140.308 121.412) (width 0.25) (layer B.Cu) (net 11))
 (segment (start 140.308 121.412) (end 141.0793 120.6407) (width 0.25) (layer B.Cu) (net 11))
 (segment (start 141.0793 120.6407) (end 141.0793 117.0312) (width 0.25) (layer B.Cu) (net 11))
 (segment (start 141.0793 117.0312) (end 140.2354 116.1873) (width 0.25) (layer B.Cu) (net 11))
 (segment (start 140.2354 116.1873) (end 139.954 116.1873) (width 0.25) (layer B.Cu) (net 11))
 (segment (start 139.954 112.522) (end 138.8287 112.522) (width 0.25) (layer F.Cu) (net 13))
 (segment (start 132.69 120.745) (end 132.69 119.5697) (width 0.25) (layer F.Cu) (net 13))
 (segment (start 132.69 119.5697) (end 133.0574 119.5697) (width 0.25) (layer F.Cu) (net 13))
 (segment (start 133.0574 119.5697) (end 133.8653 118.7618) (width 0.25) (layer F.Cu) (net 13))
 (segment (start 133.8653 118.7618) (end 133.8653 117.905) (width 0.25) (layer F.Cu) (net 13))
 (segment (start 133.8653 117.905) (end 134.8353 116.935) (width 0.25) (layer F.Cu) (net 13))
 (segment (start 134.8353 116.935) (end 135.6297 116.935) (width 0.25) (layer F.Cu) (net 13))
 (segment (start 135.6297 116.935) (end 138.8287 113.736) (width 0.25) (layer F.Cu) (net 13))
 (segment (start 138.8287 113.736) (end 138.8287 112.522) (width 0.25) (layer F.Cu) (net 13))
 (segment (start 139.954 120.142) (end 138.8287 120.142) (width 0.25) (layer B.Cu) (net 7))
 (segment (start 135.23 118.205) (end 136.8917 118.205) (width 0.25) (layer B.Cu) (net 7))
 (segment (start 136.8917 118.205) (end 138.8287 120.142) (width 0.25) (layer B.Cu) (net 7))
 (segment (start 139.954 109.982) (end 139.954 111.1073) (width 0.25) (layer B.Cu) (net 15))
 (segment (start 132.69 118.205) (end 133.8653 118.205) (width 0.25) (layer B.Cu) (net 15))
 (segment (start 133.8653 118.205) (end 133.8653 117.8376) (width 0.25) (layer B.Cu) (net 15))
 (segment (start 133.8653 117.8376) (end 134.6732 117.0297) (width 0.25) (layer B.Cu) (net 15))
 (segment (start 134.6732 117.0297) (end 135.5465 117.0297) (width 0.25) (layer B.Cu) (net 15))
 (segment (start 135.5465 117.0297) (end 138.8287 113.7475) (width 0.25) (layer B.Cu) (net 15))
 (segment (start 138.8287 113.7475) (end 138.8287 111.9512) (width 0.25) (layer B.Cu) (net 15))
 (segment (start 138.8287 111.9512) (end 139.6726 111.1073) (width 0.25) (layer B.Cu) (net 15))
 (segment (start 139.6726 111.1073) (end 139.954 111.1073) (width 0.25) (layer B.Cu) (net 15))
 (segment (start 139.954 107.442) (end 139.954 108.5673) (width 0.25) (layer B.Cu) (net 17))
 (segment (start 132.69 115.665) (end 132.69 114.4897) (width 0.25) (layer B.Cu) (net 17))
 (segment (start 132.69 114.4897) (end 133.0574 114.4897) (width 0.25) (layer B.Cu) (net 17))
 (segment (start 133.0574 114.4897) (end 133.8653 113.6818) (width 0.25) (layer B.Cu) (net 17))
 (segment (start 133.8653 113.6818) (end 133.8653 112.786) (width 0.25) (layer B.Cu) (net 17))
 (segment (start 133.8653 112.786) (end 134.7963 111.855) (width 0.25) (layer B.Cu) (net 17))
 (segment (start 134.7963 111.855) (end 135.7014 111.855) (width 0.25) (layer B.Cu) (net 17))
 (segment (start 135.7014 111.855) (end 138.9891 108.5673) (width 0.25) (layer B.Cu) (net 17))
 (segment (start 138.9891 108.5673) (end 139.954 108.5673) (width 0.25) (layer B.Cu) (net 17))
 (segment (start 147.193 79.756) (end 144.018 79.756) (width 0.25) (layer B.Cu) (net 22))
 (segment (start 135.23 100.425) (end 135.23 99.2497) (width 0.25) (layer F.Cu) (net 22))
 (segment (start 135.23 99.2497) (end 135.5974 99.2497) (width 0.25) (layer F.Cu) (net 22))
 (segment (start 135.5974 99.2497) (end 136.4053 98.4418) (width 0.25) (layer F.Cu) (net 22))
 (segment (start 136.4053 98.4418) (end 136.4053 87.3687) (width 0.25) (layer F.Cu) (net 22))
 (segment (start 136.4053 87.3687) (end 144.018 79.756) (width 0.25) (layer F.Cu) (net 22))
 (segment (start 139.954 127.762) (end 139.954 126.6367) (width 0.25) (layer F.Cu) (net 1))
 (segment (start 132.69 80.105) (end 132.69 81.2803) (width 0.25) (layer F.Cu) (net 1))
 (segment (start 132.69 81.2803) (end 133.0574 81.2803) (width 0.25) (layer F.Cu) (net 1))
 (segment (start 133.0574 81.2803) (end 133.8653 82.0882) (width 0.25) (layer F.Cu) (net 1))
 (segment (start 133.8653 82.0882) (end 133.8653 105.8204) (width 0.25) (layer F.Cu) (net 1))
 (segment (start 133.8653 105.8204) (end 134.8121 106.7672) (width 0.25) (layer F.Cu) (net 1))
 (segment (start 134.8121 106.7672) (end 135.6719 106.7672) (width 0.25) (layer F.Cu) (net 1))
 (segment (start 135.6719 106.7672) (end 138.1971 109.2924) (width 0.25) (layer F.Cu) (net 1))
 (segment (start 138.1971 109.2924) (end 138.1971 109.8283) (width 0.25) (layer F.Cu) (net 1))
 (segment (start 138.1971 109.8283) (end 139.6208 111.252) (width 0.25) (layer F.Cu) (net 1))
 (segment (start 139.6208 111.252) (end 140.3501 111.252) (width 0.25) (layer F.Cu) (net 1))
 (segment (start 140.3501 111.252) (end 141.0793 111.9812) (width 0.25) (layer F.Cu) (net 1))
 (segment (start 141.0793 111.9812) (end 141.0793 125.7928) (width 0.25) (layer F.Cu) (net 1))
 (segment (start 141.0793 125.7928) (end 140.2354 126.6367) (width 0.25) (layer F.Cu) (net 1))
 (segment (start 140.2354 126.6367) (end 139.954 126.6367) (width 0.25) (layer F.Cu) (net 1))
 (segment (start 144.018 89.916) (end 140.843 89.916) (width 0.25) (layer B.Cu) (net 21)))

